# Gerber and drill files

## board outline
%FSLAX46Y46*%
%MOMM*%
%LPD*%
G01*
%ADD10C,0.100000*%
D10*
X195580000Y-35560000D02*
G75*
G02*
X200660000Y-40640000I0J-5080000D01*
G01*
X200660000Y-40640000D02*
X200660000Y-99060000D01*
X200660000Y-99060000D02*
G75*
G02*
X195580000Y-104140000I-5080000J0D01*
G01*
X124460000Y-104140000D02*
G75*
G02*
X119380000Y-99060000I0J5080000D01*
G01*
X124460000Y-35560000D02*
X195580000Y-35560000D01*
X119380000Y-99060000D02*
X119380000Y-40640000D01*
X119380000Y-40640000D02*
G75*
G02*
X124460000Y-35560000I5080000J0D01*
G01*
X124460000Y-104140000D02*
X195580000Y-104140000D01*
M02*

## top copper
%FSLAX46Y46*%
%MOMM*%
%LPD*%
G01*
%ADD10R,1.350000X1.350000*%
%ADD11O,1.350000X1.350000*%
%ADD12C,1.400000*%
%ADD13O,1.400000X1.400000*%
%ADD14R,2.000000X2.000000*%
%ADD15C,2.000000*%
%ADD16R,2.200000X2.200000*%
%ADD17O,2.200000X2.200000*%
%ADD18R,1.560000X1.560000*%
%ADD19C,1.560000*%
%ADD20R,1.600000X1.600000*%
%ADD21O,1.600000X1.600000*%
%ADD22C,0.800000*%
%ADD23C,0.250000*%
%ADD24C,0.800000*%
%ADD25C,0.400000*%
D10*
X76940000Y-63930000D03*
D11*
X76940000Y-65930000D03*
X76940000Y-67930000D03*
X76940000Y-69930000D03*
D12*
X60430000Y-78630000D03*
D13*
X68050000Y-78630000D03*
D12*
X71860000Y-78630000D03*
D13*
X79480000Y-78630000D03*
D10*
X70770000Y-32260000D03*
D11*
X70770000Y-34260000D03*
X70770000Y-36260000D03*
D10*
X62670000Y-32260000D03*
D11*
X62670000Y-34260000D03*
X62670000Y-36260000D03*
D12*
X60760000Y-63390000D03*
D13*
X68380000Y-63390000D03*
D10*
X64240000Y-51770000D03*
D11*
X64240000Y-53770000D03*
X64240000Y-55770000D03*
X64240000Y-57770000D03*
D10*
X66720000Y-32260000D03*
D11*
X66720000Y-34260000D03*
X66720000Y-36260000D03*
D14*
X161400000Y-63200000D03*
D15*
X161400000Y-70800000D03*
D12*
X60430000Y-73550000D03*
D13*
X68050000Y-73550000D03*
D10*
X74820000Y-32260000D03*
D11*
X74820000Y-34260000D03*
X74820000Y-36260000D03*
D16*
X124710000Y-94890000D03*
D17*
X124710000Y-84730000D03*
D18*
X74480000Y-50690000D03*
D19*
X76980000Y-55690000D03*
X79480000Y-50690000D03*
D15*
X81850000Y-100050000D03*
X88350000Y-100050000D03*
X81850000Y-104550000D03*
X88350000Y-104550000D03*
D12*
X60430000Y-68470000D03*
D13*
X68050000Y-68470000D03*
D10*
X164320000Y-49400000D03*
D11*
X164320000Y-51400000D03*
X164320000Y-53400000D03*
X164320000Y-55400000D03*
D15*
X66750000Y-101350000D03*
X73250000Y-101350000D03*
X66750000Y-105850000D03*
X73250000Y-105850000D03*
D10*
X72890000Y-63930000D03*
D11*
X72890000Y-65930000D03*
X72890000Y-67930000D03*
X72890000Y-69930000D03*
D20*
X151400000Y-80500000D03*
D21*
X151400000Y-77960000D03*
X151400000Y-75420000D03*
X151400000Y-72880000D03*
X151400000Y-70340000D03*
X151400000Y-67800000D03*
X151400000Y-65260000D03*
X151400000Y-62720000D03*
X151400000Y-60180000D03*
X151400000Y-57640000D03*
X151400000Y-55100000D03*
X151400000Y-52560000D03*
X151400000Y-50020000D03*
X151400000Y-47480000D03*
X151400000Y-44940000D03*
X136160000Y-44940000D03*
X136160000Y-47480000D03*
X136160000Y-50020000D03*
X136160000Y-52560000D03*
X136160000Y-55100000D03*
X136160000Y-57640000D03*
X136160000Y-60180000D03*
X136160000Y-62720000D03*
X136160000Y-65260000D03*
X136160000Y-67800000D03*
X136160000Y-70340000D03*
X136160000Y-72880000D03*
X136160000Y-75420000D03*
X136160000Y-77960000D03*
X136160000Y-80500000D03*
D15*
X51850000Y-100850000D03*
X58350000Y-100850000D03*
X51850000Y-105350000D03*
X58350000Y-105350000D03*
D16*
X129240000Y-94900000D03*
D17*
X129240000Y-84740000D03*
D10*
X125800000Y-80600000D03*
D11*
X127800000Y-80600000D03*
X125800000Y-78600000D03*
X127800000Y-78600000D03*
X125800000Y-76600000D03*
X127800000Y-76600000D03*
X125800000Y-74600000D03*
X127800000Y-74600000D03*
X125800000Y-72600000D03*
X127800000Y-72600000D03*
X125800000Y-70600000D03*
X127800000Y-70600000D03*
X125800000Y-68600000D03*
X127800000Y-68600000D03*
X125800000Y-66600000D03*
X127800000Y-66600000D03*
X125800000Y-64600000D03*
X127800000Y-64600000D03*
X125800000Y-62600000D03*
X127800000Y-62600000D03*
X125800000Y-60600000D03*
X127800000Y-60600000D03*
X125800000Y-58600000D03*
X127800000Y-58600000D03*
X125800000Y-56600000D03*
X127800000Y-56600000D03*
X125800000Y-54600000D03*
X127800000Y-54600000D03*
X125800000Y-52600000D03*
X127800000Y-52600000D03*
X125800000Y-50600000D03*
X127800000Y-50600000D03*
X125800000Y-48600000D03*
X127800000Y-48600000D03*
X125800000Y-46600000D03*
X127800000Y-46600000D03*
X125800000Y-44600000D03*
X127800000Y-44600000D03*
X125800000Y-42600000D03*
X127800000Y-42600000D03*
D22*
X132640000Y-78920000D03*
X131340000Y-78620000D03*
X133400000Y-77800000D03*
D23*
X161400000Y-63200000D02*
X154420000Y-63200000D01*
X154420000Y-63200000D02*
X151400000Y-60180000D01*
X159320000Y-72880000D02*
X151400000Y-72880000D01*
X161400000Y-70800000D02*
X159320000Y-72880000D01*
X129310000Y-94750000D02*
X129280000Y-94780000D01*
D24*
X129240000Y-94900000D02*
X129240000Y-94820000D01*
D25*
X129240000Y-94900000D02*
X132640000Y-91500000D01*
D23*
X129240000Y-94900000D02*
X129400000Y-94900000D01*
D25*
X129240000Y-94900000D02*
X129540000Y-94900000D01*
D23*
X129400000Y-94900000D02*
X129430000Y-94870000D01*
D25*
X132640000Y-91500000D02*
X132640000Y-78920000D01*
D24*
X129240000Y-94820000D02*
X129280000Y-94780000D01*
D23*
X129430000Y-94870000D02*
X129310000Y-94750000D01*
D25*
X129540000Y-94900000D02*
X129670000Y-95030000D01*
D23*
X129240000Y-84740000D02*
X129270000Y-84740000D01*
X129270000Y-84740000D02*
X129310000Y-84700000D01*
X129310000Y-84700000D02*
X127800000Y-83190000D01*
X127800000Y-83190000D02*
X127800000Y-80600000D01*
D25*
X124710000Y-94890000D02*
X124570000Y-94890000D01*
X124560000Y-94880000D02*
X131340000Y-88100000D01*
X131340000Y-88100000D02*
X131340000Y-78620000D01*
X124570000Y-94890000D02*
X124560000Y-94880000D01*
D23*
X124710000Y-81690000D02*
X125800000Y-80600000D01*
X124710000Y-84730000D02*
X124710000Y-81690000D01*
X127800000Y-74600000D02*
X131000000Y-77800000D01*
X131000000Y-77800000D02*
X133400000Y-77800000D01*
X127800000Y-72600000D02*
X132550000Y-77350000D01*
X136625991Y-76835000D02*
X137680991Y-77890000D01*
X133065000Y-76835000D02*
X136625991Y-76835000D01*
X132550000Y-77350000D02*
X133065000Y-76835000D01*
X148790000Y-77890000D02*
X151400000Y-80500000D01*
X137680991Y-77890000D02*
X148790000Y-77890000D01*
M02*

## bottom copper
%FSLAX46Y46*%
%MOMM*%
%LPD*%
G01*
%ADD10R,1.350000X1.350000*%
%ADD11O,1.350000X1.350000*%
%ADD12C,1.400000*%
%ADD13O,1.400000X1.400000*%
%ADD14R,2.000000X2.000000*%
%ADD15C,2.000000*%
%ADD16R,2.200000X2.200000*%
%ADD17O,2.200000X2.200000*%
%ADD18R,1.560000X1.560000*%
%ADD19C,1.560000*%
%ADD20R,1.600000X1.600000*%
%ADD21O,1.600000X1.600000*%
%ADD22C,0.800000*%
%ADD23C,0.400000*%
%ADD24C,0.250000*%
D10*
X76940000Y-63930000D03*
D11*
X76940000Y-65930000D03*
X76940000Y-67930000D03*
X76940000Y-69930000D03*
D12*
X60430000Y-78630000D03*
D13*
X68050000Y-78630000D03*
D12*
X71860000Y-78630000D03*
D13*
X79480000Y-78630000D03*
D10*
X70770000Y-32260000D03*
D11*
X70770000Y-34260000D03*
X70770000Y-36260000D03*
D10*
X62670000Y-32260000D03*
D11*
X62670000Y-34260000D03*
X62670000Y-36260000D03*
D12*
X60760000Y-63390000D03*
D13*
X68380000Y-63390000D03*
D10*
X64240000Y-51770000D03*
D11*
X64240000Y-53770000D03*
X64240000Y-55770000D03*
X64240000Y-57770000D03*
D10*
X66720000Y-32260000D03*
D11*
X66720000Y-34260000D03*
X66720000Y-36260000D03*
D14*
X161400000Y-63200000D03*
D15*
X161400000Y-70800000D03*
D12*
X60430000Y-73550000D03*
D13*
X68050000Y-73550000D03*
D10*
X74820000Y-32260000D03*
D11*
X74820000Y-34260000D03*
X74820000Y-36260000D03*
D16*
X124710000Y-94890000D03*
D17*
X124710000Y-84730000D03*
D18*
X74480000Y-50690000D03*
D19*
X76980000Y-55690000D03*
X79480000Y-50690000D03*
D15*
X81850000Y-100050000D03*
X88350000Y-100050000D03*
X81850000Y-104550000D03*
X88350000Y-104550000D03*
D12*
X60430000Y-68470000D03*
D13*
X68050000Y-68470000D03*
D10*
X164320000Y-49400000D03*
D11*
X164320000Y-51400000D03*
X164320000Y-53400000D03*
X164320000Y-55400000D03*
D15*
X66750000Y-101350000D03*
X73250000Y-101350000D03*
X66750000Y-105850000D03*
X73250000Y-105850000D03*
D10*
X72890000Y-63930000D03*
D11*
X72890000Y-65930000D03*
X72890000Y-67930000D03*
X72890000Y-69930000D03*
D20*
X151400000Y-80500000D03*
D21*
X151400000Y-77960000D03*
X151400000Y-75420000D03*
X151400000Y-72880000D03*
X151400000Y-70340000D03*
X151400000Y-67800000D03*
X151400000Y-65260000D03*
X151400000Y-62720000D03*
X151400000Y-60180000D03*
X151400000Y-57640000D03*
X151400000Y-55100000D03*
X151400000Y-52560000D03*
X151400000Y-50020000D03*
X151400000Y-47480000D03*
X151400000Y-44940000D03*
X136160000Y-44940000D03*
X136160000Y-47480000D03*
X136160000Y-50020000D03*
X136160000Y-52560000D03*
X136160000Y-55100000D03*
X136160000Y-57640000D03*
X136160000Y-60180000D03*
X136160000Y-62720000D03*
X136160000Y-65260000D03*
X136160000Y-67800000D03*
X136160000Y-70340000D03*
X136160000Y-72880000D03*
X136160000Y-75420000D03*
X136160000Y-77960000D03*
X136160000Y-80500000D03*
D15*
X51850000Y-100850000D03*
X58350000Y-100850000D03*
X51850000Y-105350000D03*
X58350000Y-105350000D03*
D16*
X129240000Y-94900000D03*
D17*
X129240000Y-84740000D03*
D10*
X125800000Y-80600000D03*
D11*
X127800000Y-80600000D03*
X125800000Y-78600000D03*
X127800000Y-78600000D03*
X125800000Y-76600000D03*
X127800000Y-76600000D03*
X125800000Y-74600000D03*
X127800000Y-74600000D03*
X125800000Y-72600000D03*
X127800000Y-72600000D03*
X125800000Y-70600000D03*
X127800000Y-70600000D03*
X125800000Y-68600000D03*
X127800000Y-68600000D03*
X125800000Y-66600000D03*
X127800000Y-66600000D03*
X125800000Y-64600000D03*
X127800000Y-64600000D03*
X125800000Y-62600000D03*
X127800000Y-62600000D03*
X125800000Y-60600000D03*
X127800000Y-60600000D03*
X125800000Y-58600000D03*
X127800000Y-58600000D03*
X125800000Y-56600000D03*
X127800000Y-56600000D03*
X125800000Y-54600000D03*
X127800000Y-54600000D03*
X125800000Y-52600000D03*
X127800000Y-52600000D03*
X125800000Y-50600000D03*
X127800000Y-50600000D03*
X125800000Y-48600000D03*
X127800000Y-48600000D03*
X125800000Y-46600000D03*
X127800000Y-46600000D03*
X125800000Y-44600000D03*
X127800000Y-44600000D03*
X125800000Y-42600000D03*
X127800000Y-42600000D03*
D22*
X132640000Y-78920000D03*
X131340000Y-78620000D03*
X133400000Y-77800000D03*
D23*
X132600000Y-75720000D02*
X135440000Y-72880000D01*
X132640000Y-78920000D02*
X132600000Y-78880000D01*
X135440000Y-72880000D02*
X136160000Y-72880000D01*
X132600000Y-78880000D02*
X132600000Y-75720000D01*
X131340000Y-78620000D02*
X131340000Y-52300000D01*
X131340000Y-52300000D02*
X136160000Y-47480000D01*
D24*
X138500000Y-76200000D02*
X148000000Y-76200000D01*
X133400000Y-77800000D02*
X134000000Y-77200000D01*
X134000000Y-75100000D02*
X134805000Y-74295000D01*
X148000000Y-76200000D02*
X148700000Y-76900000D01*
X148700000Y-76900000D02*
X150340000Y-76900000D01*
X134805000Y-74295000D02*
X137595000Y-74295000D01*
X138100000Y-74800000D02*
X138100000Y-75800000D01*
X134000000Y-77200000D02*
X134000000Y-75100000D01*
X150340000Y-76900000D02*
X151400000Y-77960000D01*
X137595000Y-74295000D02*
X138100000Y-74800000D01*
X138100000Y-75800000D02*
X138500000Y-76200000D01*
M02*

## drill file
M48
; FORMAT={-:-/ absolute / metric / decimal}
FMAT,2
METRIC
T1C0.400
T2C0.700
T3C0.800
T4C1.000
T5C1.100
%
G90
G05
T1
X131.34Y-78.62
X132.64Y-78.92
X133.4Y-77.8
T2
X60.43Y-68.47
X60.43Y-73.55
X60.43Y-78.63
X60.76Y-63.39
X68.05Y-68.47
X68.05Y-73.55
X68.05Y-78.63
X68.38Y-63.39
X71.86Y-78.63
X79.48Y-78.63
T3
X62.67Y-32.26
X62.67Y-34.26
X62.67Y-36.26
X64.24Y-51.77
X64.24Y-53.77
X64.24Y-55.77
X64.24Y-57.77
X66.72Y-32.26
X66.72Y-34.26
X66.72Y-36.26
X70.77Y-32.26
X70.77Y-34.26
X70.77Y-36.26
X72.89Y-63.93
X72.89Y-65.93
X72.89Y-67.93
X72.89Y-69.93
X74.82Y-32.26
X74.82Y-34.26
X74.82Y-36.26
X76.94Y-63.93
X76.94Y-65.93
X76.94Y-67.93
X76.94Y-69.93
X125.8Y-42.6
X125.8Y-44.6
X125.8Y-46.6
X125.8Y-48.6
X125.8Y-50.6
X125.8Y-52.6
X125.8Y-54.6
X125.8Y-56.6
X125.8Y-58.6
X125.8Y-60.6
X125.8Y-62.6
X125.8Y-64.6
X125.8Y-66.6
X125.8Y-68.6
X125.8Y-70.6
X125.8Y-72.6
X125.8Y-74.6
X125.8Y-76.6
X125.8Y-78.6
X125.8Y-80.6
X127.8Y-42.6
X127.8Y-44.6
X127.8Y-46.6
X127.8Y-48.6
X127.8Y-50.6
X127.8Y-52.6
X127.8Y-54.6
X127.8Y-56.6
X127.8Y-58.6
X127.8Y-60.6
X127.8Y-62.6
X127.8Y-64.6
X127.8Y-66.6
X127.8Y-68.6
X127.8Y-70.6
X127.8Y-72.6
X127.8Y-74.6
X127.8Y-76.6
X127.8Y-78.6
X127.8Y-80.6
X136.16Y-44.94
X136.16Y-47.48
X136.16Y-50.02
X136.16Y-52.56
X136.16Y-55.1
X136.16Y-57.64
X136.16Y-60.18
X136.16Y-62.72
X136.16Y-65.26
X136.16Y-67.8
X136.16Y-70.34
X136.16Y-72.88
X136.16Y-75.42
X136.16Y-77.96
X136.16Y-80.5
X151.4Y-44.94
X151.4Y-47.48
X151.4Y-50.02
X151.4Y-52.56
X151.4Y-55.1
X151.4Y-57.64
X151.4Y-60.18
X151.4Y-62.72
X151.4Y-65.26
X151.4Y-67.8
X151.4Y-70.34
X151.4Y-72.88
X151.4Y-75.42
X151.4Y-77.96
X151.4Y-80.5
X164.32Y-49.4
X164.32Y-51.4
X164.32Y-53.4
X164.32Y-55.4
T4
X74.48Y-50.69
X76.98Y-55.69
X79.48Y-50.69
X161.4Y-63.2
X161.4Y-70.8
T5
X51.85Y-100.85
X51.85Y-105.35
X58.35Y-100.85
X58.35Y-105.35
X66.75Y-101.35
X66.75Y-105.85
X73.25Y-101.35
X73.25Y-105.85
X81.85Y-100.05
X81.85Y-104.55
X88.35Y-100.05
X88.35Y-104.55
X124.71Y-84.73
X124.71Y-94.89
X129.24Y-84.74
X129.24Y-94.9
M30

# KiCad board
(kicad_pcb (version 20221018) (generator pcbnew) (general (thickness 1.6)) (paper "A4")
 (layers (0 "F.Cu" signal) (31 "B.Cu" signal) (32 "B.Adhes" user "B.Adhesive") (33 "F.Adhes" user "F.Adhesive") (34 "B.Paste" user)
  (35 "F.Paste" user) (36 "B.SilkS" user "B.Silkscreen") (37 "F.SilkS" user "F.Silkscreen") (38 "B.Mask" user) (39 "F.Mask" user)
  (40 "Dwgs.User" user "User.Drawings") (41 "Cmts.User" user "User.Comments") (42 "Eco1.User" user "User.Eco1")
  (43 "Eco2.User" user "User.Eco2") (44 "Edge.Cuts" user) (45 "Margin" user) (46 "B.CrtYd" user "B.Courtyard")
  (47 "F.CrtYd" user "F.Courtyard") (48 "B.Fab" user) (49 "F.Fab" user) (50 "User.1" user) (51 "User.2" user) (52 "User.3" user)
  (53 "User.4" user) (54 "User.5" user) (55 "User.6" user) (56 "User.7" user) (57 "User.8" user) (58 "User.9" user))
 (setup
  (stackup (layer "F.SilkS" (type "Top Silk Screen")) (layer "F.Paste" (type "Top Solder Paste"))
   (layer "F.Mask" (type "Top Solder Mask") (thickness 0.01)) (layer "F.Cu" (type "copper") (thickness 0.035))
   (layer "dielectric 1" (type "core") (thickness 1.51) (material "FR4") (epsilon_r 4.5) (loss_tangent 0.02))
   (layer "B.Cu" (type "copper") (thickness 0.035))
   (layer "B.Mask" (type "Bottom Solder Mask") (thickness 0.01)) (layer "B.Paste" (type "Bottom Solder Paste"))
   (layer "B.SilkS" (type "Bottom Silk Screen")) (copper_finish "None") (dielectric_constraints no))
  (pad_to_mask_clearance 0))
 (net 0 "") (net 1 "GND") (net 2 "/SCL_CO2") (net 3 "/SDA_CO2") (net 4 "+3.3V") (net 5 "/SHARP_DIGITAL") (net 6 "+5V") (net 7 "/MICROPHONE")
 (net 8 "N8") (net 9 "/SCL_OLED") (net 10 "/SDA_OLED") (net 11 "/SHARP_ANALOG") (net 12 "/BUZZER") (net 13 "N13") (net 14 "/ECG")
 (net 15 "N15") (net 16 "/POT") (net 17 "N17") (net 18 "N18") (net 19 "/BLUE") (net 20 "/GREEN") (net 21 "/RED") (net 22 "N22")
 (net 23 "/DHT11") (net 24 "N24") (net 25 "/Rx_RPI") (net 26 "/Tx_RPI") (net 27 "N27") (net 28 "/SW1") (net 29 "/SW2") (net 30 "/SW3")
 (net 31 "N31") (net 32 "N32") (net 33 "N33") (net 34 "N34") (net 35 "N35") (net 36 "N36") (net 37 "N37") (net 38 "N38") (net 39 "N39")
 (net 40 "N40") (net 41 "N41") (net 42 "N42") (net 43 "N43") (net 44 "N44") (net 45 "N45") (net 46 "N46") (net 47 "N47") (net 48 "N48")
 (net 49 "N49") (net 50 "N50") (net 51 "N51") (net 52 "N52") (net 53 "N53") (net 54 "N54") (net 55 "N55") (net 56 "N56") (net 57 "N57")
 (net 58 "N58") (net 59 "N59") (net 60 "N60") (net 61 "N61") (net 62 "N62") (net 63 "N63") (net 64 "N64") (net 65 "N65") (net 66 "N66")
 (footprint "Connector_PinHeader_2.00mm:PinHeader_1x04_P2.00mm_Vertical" (layer "F.Cu") (at 76.94 63.93)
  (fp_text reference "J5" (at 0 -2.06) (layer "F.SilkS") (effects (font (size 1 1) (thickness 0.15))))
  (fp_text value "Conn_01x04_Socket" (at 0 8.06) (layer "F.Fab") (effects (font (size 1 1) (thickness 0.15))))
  (pad "1" thru_hole rect (at 0 0) (size 1.35 1.35) (drill 0.8) (layers "*.Cu" "*.Mask") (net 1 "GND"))
  (pad "2" thru_hole oval (at 0 2) (size 1.35 1.35) (drill 0.8) (layers "*.Cu" "*.Mask") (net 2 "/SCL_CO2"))
  (pad "3" thru_hole oval (at 0 4) (size 1.35 1.35) (drill 0.8) (layers "*.Cu" "*.Mask") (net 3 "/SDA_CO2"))
  (pad "4" thru_hole oval (at 0 6) (size 1.35 1.35) (drill 0.8) (layers "*.Cu" "*.Mask") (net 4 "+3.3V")))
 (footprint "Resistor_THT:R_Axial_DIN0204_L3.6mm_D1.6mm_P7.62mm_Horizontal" (layer "F.Cu") (at 60.43 78.63)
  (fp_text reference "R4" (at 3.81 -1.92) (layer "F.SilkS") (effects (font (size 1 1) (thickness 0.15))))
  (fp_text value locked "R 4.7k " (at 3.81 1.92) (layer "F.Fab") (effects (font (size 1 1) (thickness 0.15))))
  (pad "1" thru_hole circle (at 0 0) (size 1.4 1.4) (drill 0.7) (layers "*.Cu" "*.Mask") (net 2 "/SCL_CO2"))
  (pad "2" thru_hole oval (at 7.62 0) (size 1.4 1.4) (drill 0.7) (layers "*.Cu" "*.Mask") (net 4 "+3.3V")))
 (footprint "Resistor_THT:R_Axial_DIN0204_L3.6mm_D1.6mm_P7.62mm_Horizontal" (layer "F.Cu") (at 71.86 78.63)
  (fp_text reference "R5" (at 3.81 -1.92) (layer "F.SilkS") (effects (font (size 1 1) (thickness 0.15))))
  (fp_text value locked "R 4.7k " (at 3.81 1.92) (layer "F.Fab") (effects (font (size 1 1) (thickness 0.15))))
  (pad "1" thru_hole circle (at 0 0) (size 1.4 1.4) (drill 0.7) (layers "*.Cu" "*.Mask") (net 3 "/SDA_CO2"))
  (pad "2" thru_hole oval (at 7.62 0) (size 1.4 1.4) (drill 0.7) (layers "*.Cu" "*.Mask") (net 4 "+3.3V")))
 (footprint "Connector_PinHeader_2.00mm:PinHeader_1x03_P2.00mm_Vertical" (layer "F.Cu") (at 70.77 32.26)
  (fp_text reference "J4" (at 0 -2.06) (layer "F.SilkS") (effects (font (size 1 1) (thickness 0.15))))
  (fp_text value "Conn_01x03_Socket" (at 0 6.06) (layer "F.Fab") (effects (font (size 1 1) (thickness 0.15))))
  (pad "1" thru_hole rect (at 0 0) (size 1.35 1.35) (drill 0.8) (layers "*.Cu" "*.Mask") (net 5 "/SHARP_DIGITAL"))
  (pad "2" thru_hole oval (at 0 2) (size 1.35 1.35) (drill 0.8) (layers "*.Cu" "*.Mask") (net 4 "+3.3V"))
  (pad "3" thru_hole oval (at 0 4) (size 1.35 1.35) (drill 0.8) (layers "*.Cu" "*.Mask") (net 1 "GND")))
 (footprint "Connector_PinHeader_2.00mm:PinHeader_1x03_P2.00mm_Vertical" (layer "F.Cu") (at 62.67 32.26)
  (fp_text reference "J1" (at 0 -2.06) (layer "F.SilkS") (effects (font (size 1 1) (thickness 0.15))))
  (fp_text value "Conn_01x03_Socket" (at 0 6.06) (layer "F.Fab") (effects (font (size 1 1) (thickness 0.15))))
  (pad "1" thru_hole rect (at 0 0) (size 1.35 1.35) (drill 0.8) (layers "*.Cu" "*.Mask") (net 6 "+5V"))
  (pad "2" thru_hole oval (at 0 2) (size 1.35 1.35) (drill 0.8) (layers "*.Cu" "*.Mask") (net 1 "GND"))
  (pad "3" thru_hole oval (at 0 4) (size 1.35 1.35) (drill 0.8) (layers "*.Cu" "*.Mask") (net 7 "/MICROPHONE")))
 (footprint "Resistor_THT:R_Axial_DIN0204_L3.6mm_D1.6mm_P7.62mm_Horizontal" (layer "F.Cu") (at 60.76 63.39)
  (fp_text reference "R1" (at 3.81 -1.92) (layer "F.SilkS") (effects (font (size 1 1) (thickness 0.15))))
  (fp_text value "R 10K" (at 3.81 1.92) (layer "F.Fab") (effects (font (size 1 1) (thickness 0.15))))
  (pad "1" thru_hole circle (at 0 0) (size 1.4 1.4) (drill 0.7) (layers "*.Cu" "*.Mask") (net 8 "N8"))
  (pad "2" thru_hole oval (at 7.62 0) (size 1.4 1.4) (drill 0.7) (layers "*.Cu" "*.Mask") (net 1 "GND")))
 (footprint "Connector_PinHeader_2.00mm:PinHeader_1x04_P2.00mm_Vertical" (layer "F.Cu") (at 64.24 51.77)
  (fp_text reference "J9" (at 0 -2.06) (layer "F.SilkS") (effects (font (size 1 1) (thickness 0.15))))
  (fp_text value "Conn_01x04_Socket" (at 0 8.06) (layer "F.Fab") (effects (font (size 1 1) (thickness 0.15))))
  (pad "1" thru_hole rect (at 0 0) (size 1.35 1.35) (drill 0.8) (layers "*.Cu" "*.Mask") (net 4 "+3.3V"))
  (pad "2" thru_hole oval (at 0 2) (size 1.35 1.35) (drill 0.8) (layers "*.Cu" "*.Mask") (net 1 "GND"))
  (pad "3" thru_hole oval (at 0 4) (size 1.35 1.35) (drill 0.8) (layers "*.Cu" "*.Mask") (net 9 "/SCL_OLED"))
  (pad "4" thru_hole oval (at 0 6) (size 1.35 1.35) (drill 0.8) (layers "*.Cu" "*.Mask") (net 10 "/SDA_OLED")))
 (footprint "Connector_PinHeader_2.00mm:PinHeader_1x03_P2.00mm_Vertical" (layer "F.Cu") (at 66.72 32.26)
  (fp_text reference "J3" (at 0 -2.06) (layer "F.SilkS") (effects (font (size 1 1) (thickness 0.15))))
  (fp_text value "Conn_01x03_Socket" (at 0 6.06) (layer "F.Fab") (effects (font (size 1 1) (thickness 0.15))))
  (pad "1" thru_hole rect (at 0 0) (size 1.35 1.35) (drill 0.8) (layers "*.Cu" "*.Mask") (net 1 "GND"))
  (pad "2" thru_hole oval (at 0 2) (size 1.35 1.35) (drill 0.8) (layers "*.Cu" "*.Mask") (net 4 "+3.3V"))
  (pad "3" thru_hole oval (at 0 4) (size 1.35 1.35) (drill 0.8) (layers "*.Cu" "*.Mask") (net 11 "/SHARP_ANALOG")))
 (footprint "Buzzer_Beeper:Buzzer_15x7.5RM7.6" (layer "F.Cu") (at 161.4 63.2 -90)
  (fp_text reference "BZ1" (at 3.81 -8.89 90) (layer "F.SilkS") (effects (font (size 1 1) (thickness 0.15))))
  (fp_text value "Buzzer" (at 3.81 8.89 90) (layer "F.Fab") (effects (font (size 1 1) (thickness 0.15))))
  (pad "1" thru_hole rect (at 0 0 270) (size 2 2) (drill 1) (layers "*.Cu" "*.Mask") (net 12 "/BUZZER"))
  (pad "2" thru_hole circle (at 7.6 0 270) (size 2 2) (drill 1) (layers "*.Cu" "*.Mask") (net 1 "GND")))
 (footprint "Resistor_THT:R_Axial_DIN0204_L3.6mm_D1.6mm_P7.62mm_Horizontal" (layer "F.Cu") (at 60.43 73.55)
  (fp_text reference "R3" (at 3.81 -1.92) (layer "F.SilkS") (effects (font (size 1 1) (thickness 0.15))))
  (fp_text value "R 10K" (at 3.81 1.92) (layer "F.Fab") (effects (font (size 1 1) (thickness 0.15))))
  (pad "1" thru_hole circle (at 0 0) (size 1.4 1.4) (drill 0.7) (layers "*.Cu" "*.Mask") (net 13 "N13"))
  (pad "2" thru_hole oval (at 7.62 0) (size 1.4 1.4) (drill 0.7) (layers "*.Cu" "*.Mask") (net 1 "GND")))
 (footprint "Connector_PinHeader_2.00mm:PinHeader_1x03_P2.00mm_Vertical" (layer "F.Cu") (at 74.82 32.26)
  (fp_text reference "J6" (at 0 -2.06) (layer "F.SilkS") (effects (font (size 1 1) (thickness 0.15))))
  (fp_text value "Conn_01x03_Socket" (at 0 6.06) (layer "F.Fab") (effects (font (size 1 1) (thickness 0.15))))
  (pad "1" thru_hole rect (at 0 0) (size 1.35 1.35) (drill 0.8) (layers "*.Cu" "*.Mask") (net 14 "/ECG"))
  (pad "2" thru_hole oval (at 0 2) (size 1.35 1.35) (drill 0.8) (layers "*.Cu" "*.Mask") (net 4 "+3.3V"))
  (pad "3" thru_hole oval (at 0 4) (size 1.35 1.35) (drill 0.8) (layers "*.Cu" "*.Mask") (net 1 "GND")))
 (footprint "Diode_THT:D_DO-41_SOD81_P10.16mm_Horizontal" (layer "F.Cu") (at 124.71 94.89 90)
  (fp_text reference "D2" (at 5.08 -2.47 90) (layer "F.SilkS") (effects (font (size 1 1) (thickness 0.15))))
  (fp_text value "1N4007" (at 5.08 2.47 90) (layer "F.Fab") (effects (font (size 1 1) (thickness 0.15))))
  (pad "1" thru_hole rect (at 0 0 90) (size 2.2 2.2) (drill 1.1) (layers "*.Cu" "*.Mask") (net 4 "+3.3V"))
  (pad "2" thru_hole oval (at 10.16 0 90) (size 2.2 2.2) (drill 1.1) (layers "*.Cu" "*.Mask") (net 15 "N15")))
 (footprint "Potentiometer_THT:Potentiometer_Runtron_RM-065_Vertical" (layer "F.Cu") (at 74.48 50.69)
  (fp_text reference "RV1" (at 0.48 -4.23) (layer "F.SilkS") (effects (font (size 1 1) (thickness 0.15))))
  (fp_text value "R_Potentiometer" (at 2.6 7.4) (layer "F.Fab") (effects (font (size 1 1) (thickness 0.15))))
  (pad "1" thru_hole rect (at 0 0) (size 1.56 1.56) (drill 1) (layers "*.Cu" "*.Mask") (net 6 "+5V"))
  (pad "2" thru_hole circle (at 2.5 5) (size 1.56 1.56) (drill 1) (layers "*.Cu" "*.Mask") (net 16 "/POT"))
  (pad "3" thru_hole circle (at 5 0) (size 1.56 1.56) (drill 1) (layers "*.Cu" "*.Mask") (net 1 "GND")))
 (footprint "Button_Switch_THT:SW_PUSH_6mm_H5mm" (layer "F.Cu") (at 81.85 100.05)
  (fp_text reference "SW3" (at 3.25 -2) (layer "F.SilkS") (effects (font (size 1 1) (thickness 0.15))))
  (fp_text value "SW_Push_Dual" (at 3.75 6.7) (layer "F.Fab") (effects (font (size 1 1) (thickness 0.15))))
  (pad "1" thru_hole circle (at 0 0 90) (size 2 2) (drill 1.1) (layers "*.Cu" "*.Mask") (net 6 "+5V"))
  (pad "1" thru_hole circle (at 6.5 0 90) (size 2 2) (drill 1.1) (layers "*.Cu" "*.Mask") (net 6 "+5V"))
  (pad "2" thru_hole circle (at 0 4.5 90) (size 2 2) (drill 1.1) (layers "*.Cu" "*.Mask") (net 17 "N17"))
  (pad "2" thru_hole circle (at 6.5 4.5 90) (size 2 2) (drill 1.1) (layers "*.Cu" "*.Mask") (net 17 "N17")))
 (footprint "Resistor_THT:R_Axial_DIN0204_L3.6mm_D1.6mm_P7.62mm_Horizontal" (layer "F.Cu") (at 60.43 68.47)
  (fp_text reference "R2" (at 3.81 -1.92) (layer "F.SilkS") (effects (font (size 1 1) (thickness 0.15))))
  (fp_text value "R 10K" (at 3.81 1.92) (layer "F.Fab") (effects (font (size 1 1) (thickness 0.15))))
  (pad "1" thru_hole circle (at 0 0) (size 1.4 1.4) (drill 0.7) (layers "*.Cu" "*.Mask") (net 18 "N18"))
  (pad "2" thru_hole oval (at 7.62 0) (size 1.4 1.4) (drill 0.7) (layers "*.Cu" "*.Mask") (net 1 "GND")))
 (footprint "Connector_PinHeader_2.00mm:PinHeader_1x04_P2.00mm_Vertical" (layer "F.Cu") (at 164.32 49.4)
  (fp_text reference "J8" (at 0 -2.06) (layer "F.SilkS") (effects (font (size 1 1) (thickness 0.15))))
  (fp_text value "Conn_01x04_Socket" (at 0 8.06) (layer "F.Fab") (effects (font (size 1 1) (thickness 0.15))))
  (pad "1" thru_hole rect (at 0 0) (size 1.35 1.35) (drill 0.8) (layers "*.Cu" "*.Mask") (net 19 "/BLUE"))
  (pad "2" thru_hole oval (at 0 2) (size 1.35 1.35) (drill 0.8) (layers "*.Cu" "*.Mask") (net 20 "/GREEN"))
  (pad "3" thru_hole oval (at 0 4) (size 1.35 1.35) (drill 0.8) (layers "*.Cu" "*.Mask") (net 1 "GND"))
  (pad "4" thru_hole oval (at 0 6) (size 1.35 1.35) (drill 0.8) (layers "*.Cu" "*.Mask") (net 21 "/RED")))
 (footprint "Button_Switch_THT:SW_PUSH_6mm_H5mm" (layer "F.Cu") (at 66.75 101.35)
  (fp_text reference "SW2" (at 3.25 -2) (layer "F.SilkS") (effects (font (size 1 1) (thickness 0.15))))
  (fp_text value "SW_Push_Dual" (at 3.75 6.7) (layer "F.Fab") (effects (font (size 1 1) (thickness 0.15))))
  (pad "1" thru_hole circle (at 0 0 90) (size 2 2) (drill 1.1) (layers "*.Cu" "*.Mask") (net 6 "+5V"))
  (pad "1" thru_hole circle (at 6.5 0 90) (size 2 2) (drill 1.1) (layers "*.Cu" "*.Mask") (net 6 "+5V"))
  (pad "2" thru_hole circle (at 0 4.5 90) (size 2 2) (drill 1.1) (layers "*.Cu" "*.Mask") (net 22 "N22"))
  (pad "2" thru_hole circle (at 6.5 4.5 90) (size 2 2) (drill 1.1) (layers "*.Cu" "*.Mask") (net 22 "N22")))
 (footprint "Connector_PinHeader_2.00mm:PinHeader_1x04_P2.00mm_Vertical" (layer "F.Cu") (at 72.89 63.93)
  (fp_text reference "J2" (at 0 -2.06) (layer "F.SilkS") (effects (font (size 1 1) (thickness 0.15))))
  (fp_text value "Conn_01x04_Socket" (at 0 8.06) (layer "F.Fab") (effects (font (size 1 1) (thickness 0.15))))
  (pad "1" thru_hole rect (at 0 0) (size 1.35 1.35) (drill 0.8) (layers "*.Cu" "*.Mask") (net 6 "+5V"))
  (pad "2" thru_hole oval (at 0 2) (size 1.35 1.35) (drill 0.8) (layers "*.Cu" "*.Mask") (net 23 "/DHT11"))
  (pad "3" thru_hole oval (at 0 4) (size 1.35 1.35) (drill 0.8) (layers "*.Cu" "*.Mask") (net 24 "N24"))
  (pad "4" thru_hole oval (at 0 6) (size 1.35 1.35) (drill 0.8) (layers "*.Cu" "*.Mask") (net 1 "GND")))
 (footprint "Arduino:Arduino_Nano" (layer "F.Cu") (at 151.4 80.5 180)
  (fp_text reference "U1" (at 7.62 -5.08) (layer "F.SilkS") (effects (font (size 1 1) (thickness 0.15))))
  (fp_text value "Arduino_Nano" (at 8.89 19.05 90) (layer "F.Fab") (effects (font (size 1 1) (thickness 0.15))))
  (pad "1" thru_hole rect (at 0 0 180) (size 1.6 1.6) (drill 0.8) (layers "*.Cu" "*.Mask") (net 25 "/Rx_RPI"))
  (pad "2" thru_hole oval (at 0 2.54 180) (size 1.6 1.6) (drill 0.8) (layers "*.Cu" "*.Mask") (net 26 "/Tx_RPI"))
  (pad "3" thru_hole oval (at 0 5.08 180) (size 1.6 1.6) (drill 0.8) (layers "*.Cu" "*.Mask") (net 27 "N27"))
  (pad "4" thru_hole oval (at 0 7.62 180) (size 1.6 1.6) (drill 0.8) (layers "*.Cu" "*.Mask") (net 1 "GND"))
  (pad "5" thru_hole oval (at 0 10.16 180) (size 1.6 1.6) (drill 0.8) (layers "*.Cu" "*.Mask") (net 14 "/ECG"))
  (pad "6" thru_hole oval (at 0 12.7 180) (size 1.6 1.6) (drill 0.8) (layers "*.Cu" "*.Mask") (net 5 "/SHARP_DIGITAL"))
  (pad "7" thru_hole oval (at 0 15.24 180) (size 1.6 1.6) (drill 0.8) (layers "*.Cu" "*.Mask") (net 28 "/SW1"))
  (pad "8" thru_hole oval (at 0 17.78 180) (size 1.6 1.6) (drill 0.8) (layers "*.Cu" "*.Mask") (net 23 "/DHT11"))
  (pad "9" thru_hole oval (at 0 20.32 180) (size 1.6 1.6) (drill 0.8) (layers "*.Cu" "*.Mask") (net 12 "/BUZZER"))
  (pad "10" thru_hole oval (at 0 22.86 180) (size 1.6 1.6) (drill 0.8) (layers "*.Cu" "*.Mask") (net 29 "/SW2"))
  (pad "11" thru_hole oval (at 0 25.4 180) (size 1.6 1.6) (drill 0.8) (layers "*.Cu" "*.Mask") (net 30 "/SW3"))
  (pad "12" thru_hole oval (at 0 27.94 180) (size 1.6 1.6) (drill 0.8) (layers "*.Cu" "*.Mask") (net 19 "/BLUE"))
  (pad "13" thru_hole oval (at 0 30.48 180) (size 1.6 1.6) (drill 0.8) (layers "*.Cu" "*.Mask") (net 20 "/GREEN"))
  (pad "14" thru_hole oval (at 0 33.02 180) (size 1.6 1.6) (drill 0.8) (layers "*.Cu" "*.Mask") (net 21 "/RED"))
  (pad "15" thru_hole oval (at 0 35.56 180) (size 1.6 1.6) (drill 0.8) (layers "*.Cu" "*.Mask") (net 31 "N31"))
  (pad "16" thru_hole oval (at 15.24 35.56 180) (size 1.6 1.6) (drill 0.8) (layers "*.Cu" "*.Mask") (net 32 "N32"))
  (pad "17" thru_hole oval (at 15.24 33.02 180) (size 1.6 1.6) (drill 0.8) (layers "*.Cu" "*.Mask") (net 4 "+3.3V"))
  (pad "18" thru_hole oval (at 15.24 30.48 180) (size 1.6 1.6) (drill 0.8) (layers "*.Cu" "*.Mask") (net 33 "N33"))
  (pad "19" thru_hole oval (at 15.24 27.94 180) (size 1.6 1.6) (drill 0.8) (layers "*.Cu" "*.Mask") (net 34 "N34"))
  (pad "20" thru_hole oval (at 15.24 25.4 180) (size 1.6 1.6) (drill 0.8) (layers "*.Cu" "*.Mask") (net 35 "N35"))
  (pad "21" thru_hole oval (at 15.24 22.86 180) (size 1.6 1.6) (drill 0.8) (layers "*.Cu" "*.Mask") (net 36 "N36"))
  (pad "22" thru_hole oval (at 15.24 20.32 180) (size 1.6 1.6) (drill 0.8) (layers "*.Cu" "*.Mask") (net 7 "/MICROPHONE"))
  (pad "23" thru_hole oval (at 15.24 17.78 180) (size 1.6 1.6) (drill 0.8) (layers "*.Cu" "*.Mask") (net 3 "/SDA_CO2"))
  (pad "24" thru_hole oval (at 15.24 15.24 180) (size 1.6 1.6) (drill 0.8) (layers "*.Cu" "*.Mask") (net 2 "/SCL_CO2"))
  (pad "25" thru_hole oval (at 15.24 12.7 180) (size 1.6 1.6) (drill 0.8) (layers "*.Cu" "*.Mask") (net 11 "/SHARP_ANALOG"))
  (pad "26" thru_hole oval (at 15.24 10.16 180) (size 1.6 1.6) (drill 0.8) (layers "*.Cu" "*.Mask") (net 16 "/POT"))
  (pad "27" thru_hole oval (at 15.24 7.62 180) (size 1.6 1.6) (drill 0.8) (layers "*.Cu" "*.Mask") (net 6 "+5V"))
  (pad "28" thru_hole oval (at 15.24 5.08 180) (size 1.6 1.6) (drill 0.8) (layers "*.Cu" "*.Mask") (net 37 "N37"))
  (pad "29" thru_hole oval (at 15.24 2.54 180) (size 1.6 1.6) (drill 0.8) (layers "*.Cu" "*.Mask") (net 1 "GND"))
  (pad "30" thru_hole oval (at 15.24 0 180) (size 1.6 1.6) (drill 0.8) (layers "*.Cu" "*.Mask") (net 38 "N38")))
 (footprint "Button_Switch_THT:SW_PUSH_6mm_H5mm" (layer "F.Cu") (at 51.85 100.85)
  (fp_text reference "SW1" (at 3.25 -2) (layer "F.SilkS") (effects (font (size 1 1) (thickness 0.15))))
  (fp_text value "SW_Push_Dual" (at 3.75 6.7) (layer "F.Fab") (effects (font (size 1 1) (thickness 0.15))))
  (pad "1" thru_hole circle (at 0 0 90) (size 2 2) (drill 1.1) (layers "*.Cu" "*.Mask") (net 6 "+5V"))
  (pad "1" thru_hole circle (at 6.5 0 90) (size 2 2) (drill 1.1) (layers "*.Cu" "*.Mask") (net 6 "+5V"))
  (pad "2" thru_hole circle (at 0 4.5 90) (size 2 2) (drill 1.1) (layers "*.Cu" "*.Mask") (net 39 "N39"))
  (pad "2" thru_hole circle (at 6.5 4.5 90) (size 2 2) (drill 1.1) (layers "*.Cu" "*.Mask") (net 39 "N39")))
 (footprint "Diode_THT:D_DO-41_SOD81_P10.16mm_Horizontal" (layer "F.Cu") (at 129.24 94.9 90)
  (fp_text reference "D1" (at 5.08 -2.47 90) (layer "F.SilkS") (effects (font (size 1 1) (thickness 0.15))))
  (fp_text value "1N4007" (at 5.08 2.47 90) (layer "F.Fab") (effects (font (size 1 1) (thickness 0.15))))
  (pad "1" thru_hole rect (at 0 0 90) (size 2.2 2.2) (drill 1.1) (layers "*.Cu" "*.Mask") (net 6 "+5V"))
  (pad "2" thru_hole oval (at 10.16 0 90) (size 2.2 2.2) (drill 1.1) (layers "*.Cu" "*.Mask") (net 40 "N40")))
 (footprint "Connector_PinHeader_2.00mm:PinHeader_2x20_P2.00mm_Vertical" (layer "B.Cu") (at 125.8 80.6)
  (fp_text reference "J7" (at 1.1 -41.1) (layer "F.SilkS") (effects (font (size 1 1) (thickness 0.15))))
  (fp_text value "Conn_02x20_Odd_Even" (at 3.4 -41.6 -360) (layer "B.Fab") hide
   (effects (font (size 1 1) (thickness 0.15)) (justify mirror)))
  (pad "1" thru_hole rect (at 0 0) (size 1.35 1.35) (drill 0.8) (layers "*.Cu" "*.Mask") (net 15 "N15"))
  (pad "2" thru_hole oval (at 2 0) (size 1.35 1.35) (drill 0.8) (layers "*.Cu" "*.Mask") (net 40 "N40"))
  (pad "3" thru_hole oval (at 0 -2) (size 1.35 1.35) (drill 0.8) (layers "*.Cu" "*.Mask") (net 10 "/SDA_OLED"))
  (pad "4" thru_hole oval (at 2 -2) (size 1.35 1.35) (drill 0.8) (layers "*.Cu" "*.Mask") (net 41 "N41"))
  (pad "5" thru_hole oval (at 0 -4) (size 1.35 1.35) (drill 0.8) (layers "*.Cu" "*.Mask") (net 9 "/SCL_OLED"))
  (pad "6" thru_hole oval (at 2 -4) (size 1.35 1.35) (drill 0.8) (layers "*.Cu" "*.Mask") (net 1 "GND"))
  (pad "7" thru_hole oval (at 0 -6) (size 1.35 1.35) (drill 0.8) (layers "*.Cu" "*.Mask") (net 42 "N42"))
  (pad "8" thru_hole oval (at 2 -6) (size 1.35 1.35) (drill 0.8) (layers "*.Cu" "*.Mask") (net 26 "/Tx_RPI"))
  (pad "9" thru_hole oval (at 0 -8) (size 1.35 1.35) (drill 0.8) (layers "*.Cu" "*.Mask") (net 1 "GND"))
  (pad "10" thru_hole oval (at 2 -8) (size 1.35 1.35) (drill 0.8) (layers "*.Cu" "*.Mask") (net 25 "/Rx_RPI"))
  (pad "11" thru_hole oval (at 0 -10) (size 1.35 1.35) (drill 0.8) (layers "*.Cu" "*.Mask") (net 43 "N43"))
  (pad "12" thru_hole oval (at 2 -10) (size 1.35 1.35) (drill 0.8) (layers "*.Cu" "*.Mask") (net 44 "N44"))
  (pad "13" thru_hole oval (at 0 -12) (size 1.35 1.35) (drill 0.8) (layers "*.Cu" "*.Mask") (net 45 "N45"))
  (pad "14" thru_hole oval (at 2 -12) (size 1.35 1.35) (drill 0.8) (layers "*.Cu" "*.Mask") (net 1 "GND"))
  (pad "15" thru_hole oval (at 0 -14) (size 1.35 1.35) (drill 0.8) (layers "*.Cu" "*.Mask") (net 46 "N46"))
  (pad "16" thru_hole oval (at 2 -14) (size 1.35 1.35) (drill 0.8) (layers "*.Cu" "*.Mask") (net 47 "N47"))
  (pad "17" thru_hole oval (at 0 -16) (size 1.35 1.35) (drill 0.8) (layers "*.Cu" "*.Mask") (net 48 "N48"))
  (pad "18" thru_hole oval (at 2 -16) (size 1.35 1.35) (drill 0.8) (layers "*.Cu" "*.Mask") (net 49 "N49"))
  (pad "19" thru_hole oval (at 0 -18) (size 1.35 1.35) (drill 0.8) (layers "*.Cu" "*.Mask") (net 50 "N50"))
  (pad "20" thru_hole oval (at 2 -18) (size 1.35 1.35) (drill 0.8) (layers "*.Cu" "*.Mask") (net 1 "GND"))
  (pad "21" thru_hole oval (at 0 -20) (size 1.35 1.35) (drill 0.8) (layers "*.Cu" "*.Mask") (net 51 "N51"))
  (pad "22" thru_hole oval (at 2 -20) (size 1.35 1.35) (drill 0.8) (layers "*.Cu" "*.Mask") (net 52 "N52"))
  (pad "23" thru_hole oval (at 0 -22) (size 1.35 1.35) (drill 0.8) (layers "*.Cu" "*.Mask") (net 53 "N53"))
  (pad "24" thru_hole oval (at 2 -22) (size 1.35 1.35) (drill 0.8) (layers "*.Cu" "*.Mask") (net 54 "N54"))
  (pad "25" thru_hole oval (at 0 -24) (size 1.35 1.35) (drill 0.8) (layers "*.Cu" "*.Mask") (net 1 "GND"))
  (pad "26" thru_hole oval (at 2 -24) (size 1.35 1.35) (drill 0.8) (layers "*.Cu" "*.Mask") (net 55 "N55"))
  (pad "27" thru_hole oval (at 0 -26) (size 1.35 1.35) (drill 0.8) (layers "*.Cu" "*.Mask") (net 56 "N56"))
  (pad "28" thru_hole oval (at 2 -26) (size 1.35 1.35) (drill 0.8) (layers "*.Cu" "*.Mask") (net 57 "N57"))
  (pad "29" thru_hole oval (at 0 -28) (size 1.35 1.35) (drill 0.8) (layers "*.Cu" "*.Mask") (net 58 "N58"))
  (pad "30" thru_hole oval (at 2 -28) (size 1.35 1.35) (drill 0.8) (layers "*.Cu" "*.Mask") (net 1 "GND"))
  (pad "31" thru_hole oval (at 0 -30) (size 1.35 1.35) (drill 0.8) (layers "*.Cu" "*.Mask") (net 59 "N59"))
  (pad "32" thru_hole oval (at 2 -30) (size 1.35 1.35) (drill 0.8) (layers "*.Cu" "*.Mask") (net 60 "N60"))
  (pad "33" thru_hole oval (at 0 -32) (size 1.35 1.35) (drill 0.8) (layers "*.Cu" "*.Mask") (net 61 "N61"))
  (pad "34" thru_hole oval (at 2 -32) (size 1.35 1.35) (drill 0.8) (layers "*.Cu" "*.Mask") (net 1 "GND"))
  (pad "35" thru_hole oval (at 0 -34) (size 1.35 1.35) (drill 0.8) (layers "*.Cu" "*.Mask") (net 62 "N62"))
  (pad "36" thru_hole oval (at 2 -34) (size 1.35 1.35) (drill 0.8) (layers "*.Cu" "*.Mask") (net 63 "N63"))
  (pad "37" thru_hole oval (at 0 -36) (size 1.35 1.35) (drill 0.8) (layers "*.Cu" "*.Mask") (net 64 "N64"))
  (pad "38" thru_hole oval (at 2 -36) (size 1.35 1.35) (drill 0.8) (layers "*.Cu" "*.Mask") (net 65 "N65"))
  (pad "39" thru_hole oval (at 0 -38) (size 1.35 1.35) (drill 0.8) (layers "*.Cu" "*.Mask") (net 1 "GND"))
  (pad "40" thru_hole oval (at 2 -38) (size 1.35 1.35) (drill 0.8) (layers "*.Cu" "*.Mask") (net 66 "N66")))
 (gr_arc locked (start 195.58 35.56) (mid 199.172102 37.047898) (end 200.66 40.64) (stroke (width 0.1) (type default)) (layer "Edge.Cuts"))
 (gr_line locked (start 200.66 40.64) (end 200.66 99.06) (stroke (width 0.1) (type default)) (layer "Edge.Cuts"))
 (gr_arc locked (start 200.66 99.06) (mid 199.172102 102.652102) (end 195.58 104.14) (stroke (width 0.1) (type default)) (layer "Edge.Cuts"))
 (gr_arc locked (start 124.46 104.14) (mid 120.867898 102.652102) (end 119.38 99.06) (stroke (width 0.1) (type default)) (layer "Edge.Cuts"))
 (gr_line locked (start 124.46 35.56) (end 195.58 35.56) (stroke (width 0.1) (type default)) (layer "Edge.Cuts"))
 (gr_line locked (start 119.38 99.06) (end 119.38 40.64) (stroke (width 0.1) (type default)) (layer "Edge.Cuts"))
 (gr_arc locked (start 119.38 40.64) (mid 120.867898 37.047898) (end 124.46 35.56) (stroke (width 0.1) (type default)) (layer "Edge.Cuts"))
 (gr_line locked (start 124.46 104.14) (end 195.58 104.14) (stroke (width 0.1) (type default)) (layer "Edge.Cuts"))
 (segment (start 161.4 63.2) (end 154.42 63.2) (width 0.25) (layer "F.Cu") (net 12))
 (segment (start 154.42 63.2) (end 151.4 60.18) (width 0.25) (layer "F.Cu") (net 12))
 (segment (start 159.32 72.88) (end 151.4 72.88) (width 0.25) (layer "F.Cu") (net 1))
 (segment (start 161.4 70.8) (end 159.32 72.88) (width 0.25) (layer "F.Cu") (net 1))
 (segment (start 129.31 94.75) (end 129.28 94.78) (width 0.25) (layer "F.Cu") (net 6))
 (segment (start 129.24 94.9) (end 129.24 94.82) (width 0.8) (layer "F.Cu") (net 6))
 (segment (start 129.24 94.9) (end 132.64 91.5) (width 0.4) (layer "F.Cu") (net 6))
 (segment (start 129.24 94.9) (end 129.4 94.9) (width 0.25) (layer "F.Cu") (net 6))
 (segment (start 129.24 94.9) (end 129.54 94.9) (width 0.4) (layer "F.Cu") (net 6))
 (segment (start 129.4 94.9) (end 129.43 94.87) (width 0.25) (layer "F.Cu") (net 6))
 (segment (start 132.64 91.5) (end 132.64 78.92) (width 0.4) (layer "F.Cu") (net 6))
 (segment (start 129.24 94.82) (end 129.28 94.78) (width 0.8) (layer "F.Cu") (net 6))
 (segment (start 129.43 94.87) (end 129.31 94.75) (width 0.25) (layer "F.Cu") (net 6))
 (segment (start 129.54 94.9) (end 129.67 95.03) (width 0.4) (layer "F.Cu") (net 6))
 (via (at 132.64 78.92) (size 0.8) (drill 0.4) (layers "F.Cu" "B.Cu") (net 6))
 (segment (start 132.6 75.72) (end 135.44 72.88) (width 0.4) (layer "B.Cu") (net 6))
 (segment (start 132.64 78.92) (end 132.6 78.88) (width 0.4) (layer "B.Cu") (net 6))
 (segment (start 135.44 72.88) (end 136.16 72.88) (width 0.4) (layer "B.Cu") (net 6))
 (segment (start 132.6 78.88) (end 132.6 75.72) (width 0.4) (layer "B.Cu") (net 6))
 (segment (start 129.24 84.74) (end 129.27 84.74) (width 0.25) (layer "F.Cu") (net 40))
 (segment (start 129.27 84.74) (end 129.31 84.7) (width 0.25) (layer "F.Cu") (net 40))
 (segment (start 129.31 84.7) (end 127.8 83.19) (width 0.25) (layer "F.Cu") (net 40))
 (segment (start 127.8 83.19) (end 127.8 80.6) (width 0.25) (layer "F.Cu") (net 40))
 (segment (start 124.71 94.89) (end 124.57 94.89) (width 0.4) (layer "F.Cu") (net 4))
 (segment (start 124.56 94.88) (end 131.34 88.1) (width 0.4) (layer "F.Cu") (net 4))
 (segment (start 131.34 88.1) (end 131.34 78.62) (width 0.4) (layer "F.Cu") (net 4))
 (segment (start 124.57 94.89) (end 124.56 94.88) (width 0.4) (layer "F.Cu") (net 4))
 (via (at 131.34 78.62) (size 0.8) (drill 0.4) (layers "F.Cu" "B.Cu") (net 4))
 (segment (start 131.34 78.62) (end 131.34 52.3) (width 0.4) (layer "B.Cu") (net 4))
 (segment (start 131.34 52.3) (end 136.16 47.48) (width 0.4) (layer "B.Cu") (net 4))
 (segment (start 124.71 81.69) (end 125.8 80.6) (width 0.25) (layer "F.Cu") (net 15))
 (segment (start 124.71 84.73) (end 124.71 81.69) (width 0.25) (layer "F.Cu") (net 15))
 (segment (start 127.8 74.6) (end 131 77.8) (width 0.25) (layer "F.Cu") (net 26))
 (segment (start 131 77.8) (end 133.4 77.8) (width 0.25) (layer "F.Cu") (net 26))
 (via (at 133.4 77.8) (size 0.8) (drill 0.4) (layers "F.Cu" "B.Cu") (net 26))
 (segment (start 138.5 76.2) (end 148 76.2) (width 0.25) (layer "B.Cu") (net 26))
 (segment (start 133.4 77.8) (end 134 77.2) (width 0.25) (layer "B.Cu") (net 26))
 (segment (start 134 75.1) (end 134.805 74.295) (width 0.25) (layer "B.Cu") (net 26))
 (segment (start 148 76.2) (end 148.7 76.9) (width 0.25) (layer "B.Cu") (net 26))
 (segment (start 148.7 76.9) (end 150.34 76.9) (width 0.25) (layer "B.Cu") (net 26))
 (segment (start 134.805 74.295) (end 137.595 74.295) (width 0.25) (layer "B.Cu") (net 26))
 (segment (start 138.1 74.8) (end 138.1 75.8) (width 0.25) (layer "B.Cu") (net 26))
 (segment (start 134 77.2) (end 134 75.1) (width 0.25) (layer "B.Cu") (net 26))
 (segment (start 150.34 76.9) (end 151.4 77.96) (width 0.25) (layer "B.Cu") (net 26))
 (segment (start 137.595 74.295) (end 138.1 74.8) (width 0.25) (layer "B.Cu") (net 26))
 (segment (start 138.1 75.8) (end 138.5 76.2) (width 0.25) (layer "B.Cu") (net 26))
 (segment (start 127.8 72.6) (end 132.55 77.35) (width 0.25) (layer "F.Cu") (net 25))
 (segment (start 136.625991 76.835) (end 137.680991 77.89) (width 0.25) (layer "F.Cu") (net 25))
 (segment (start 133.065 76.835) (end 136.625991 76.835) (width 0.25) (layer "F.Cu") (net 25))
 (segment (start 132.55 77.35) (end 133.065 76.835) (width 0.25) (layer "F.Cu") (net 25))
 (segment (start 148.79 77.89) (end 151.4 80.5) (width 0.25) (layer "F.Cu") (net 25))
 (segment (start 137.680991 77.89) (end 148.79 77.89) (width 0.25) (layer "F.Cu") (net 25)))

